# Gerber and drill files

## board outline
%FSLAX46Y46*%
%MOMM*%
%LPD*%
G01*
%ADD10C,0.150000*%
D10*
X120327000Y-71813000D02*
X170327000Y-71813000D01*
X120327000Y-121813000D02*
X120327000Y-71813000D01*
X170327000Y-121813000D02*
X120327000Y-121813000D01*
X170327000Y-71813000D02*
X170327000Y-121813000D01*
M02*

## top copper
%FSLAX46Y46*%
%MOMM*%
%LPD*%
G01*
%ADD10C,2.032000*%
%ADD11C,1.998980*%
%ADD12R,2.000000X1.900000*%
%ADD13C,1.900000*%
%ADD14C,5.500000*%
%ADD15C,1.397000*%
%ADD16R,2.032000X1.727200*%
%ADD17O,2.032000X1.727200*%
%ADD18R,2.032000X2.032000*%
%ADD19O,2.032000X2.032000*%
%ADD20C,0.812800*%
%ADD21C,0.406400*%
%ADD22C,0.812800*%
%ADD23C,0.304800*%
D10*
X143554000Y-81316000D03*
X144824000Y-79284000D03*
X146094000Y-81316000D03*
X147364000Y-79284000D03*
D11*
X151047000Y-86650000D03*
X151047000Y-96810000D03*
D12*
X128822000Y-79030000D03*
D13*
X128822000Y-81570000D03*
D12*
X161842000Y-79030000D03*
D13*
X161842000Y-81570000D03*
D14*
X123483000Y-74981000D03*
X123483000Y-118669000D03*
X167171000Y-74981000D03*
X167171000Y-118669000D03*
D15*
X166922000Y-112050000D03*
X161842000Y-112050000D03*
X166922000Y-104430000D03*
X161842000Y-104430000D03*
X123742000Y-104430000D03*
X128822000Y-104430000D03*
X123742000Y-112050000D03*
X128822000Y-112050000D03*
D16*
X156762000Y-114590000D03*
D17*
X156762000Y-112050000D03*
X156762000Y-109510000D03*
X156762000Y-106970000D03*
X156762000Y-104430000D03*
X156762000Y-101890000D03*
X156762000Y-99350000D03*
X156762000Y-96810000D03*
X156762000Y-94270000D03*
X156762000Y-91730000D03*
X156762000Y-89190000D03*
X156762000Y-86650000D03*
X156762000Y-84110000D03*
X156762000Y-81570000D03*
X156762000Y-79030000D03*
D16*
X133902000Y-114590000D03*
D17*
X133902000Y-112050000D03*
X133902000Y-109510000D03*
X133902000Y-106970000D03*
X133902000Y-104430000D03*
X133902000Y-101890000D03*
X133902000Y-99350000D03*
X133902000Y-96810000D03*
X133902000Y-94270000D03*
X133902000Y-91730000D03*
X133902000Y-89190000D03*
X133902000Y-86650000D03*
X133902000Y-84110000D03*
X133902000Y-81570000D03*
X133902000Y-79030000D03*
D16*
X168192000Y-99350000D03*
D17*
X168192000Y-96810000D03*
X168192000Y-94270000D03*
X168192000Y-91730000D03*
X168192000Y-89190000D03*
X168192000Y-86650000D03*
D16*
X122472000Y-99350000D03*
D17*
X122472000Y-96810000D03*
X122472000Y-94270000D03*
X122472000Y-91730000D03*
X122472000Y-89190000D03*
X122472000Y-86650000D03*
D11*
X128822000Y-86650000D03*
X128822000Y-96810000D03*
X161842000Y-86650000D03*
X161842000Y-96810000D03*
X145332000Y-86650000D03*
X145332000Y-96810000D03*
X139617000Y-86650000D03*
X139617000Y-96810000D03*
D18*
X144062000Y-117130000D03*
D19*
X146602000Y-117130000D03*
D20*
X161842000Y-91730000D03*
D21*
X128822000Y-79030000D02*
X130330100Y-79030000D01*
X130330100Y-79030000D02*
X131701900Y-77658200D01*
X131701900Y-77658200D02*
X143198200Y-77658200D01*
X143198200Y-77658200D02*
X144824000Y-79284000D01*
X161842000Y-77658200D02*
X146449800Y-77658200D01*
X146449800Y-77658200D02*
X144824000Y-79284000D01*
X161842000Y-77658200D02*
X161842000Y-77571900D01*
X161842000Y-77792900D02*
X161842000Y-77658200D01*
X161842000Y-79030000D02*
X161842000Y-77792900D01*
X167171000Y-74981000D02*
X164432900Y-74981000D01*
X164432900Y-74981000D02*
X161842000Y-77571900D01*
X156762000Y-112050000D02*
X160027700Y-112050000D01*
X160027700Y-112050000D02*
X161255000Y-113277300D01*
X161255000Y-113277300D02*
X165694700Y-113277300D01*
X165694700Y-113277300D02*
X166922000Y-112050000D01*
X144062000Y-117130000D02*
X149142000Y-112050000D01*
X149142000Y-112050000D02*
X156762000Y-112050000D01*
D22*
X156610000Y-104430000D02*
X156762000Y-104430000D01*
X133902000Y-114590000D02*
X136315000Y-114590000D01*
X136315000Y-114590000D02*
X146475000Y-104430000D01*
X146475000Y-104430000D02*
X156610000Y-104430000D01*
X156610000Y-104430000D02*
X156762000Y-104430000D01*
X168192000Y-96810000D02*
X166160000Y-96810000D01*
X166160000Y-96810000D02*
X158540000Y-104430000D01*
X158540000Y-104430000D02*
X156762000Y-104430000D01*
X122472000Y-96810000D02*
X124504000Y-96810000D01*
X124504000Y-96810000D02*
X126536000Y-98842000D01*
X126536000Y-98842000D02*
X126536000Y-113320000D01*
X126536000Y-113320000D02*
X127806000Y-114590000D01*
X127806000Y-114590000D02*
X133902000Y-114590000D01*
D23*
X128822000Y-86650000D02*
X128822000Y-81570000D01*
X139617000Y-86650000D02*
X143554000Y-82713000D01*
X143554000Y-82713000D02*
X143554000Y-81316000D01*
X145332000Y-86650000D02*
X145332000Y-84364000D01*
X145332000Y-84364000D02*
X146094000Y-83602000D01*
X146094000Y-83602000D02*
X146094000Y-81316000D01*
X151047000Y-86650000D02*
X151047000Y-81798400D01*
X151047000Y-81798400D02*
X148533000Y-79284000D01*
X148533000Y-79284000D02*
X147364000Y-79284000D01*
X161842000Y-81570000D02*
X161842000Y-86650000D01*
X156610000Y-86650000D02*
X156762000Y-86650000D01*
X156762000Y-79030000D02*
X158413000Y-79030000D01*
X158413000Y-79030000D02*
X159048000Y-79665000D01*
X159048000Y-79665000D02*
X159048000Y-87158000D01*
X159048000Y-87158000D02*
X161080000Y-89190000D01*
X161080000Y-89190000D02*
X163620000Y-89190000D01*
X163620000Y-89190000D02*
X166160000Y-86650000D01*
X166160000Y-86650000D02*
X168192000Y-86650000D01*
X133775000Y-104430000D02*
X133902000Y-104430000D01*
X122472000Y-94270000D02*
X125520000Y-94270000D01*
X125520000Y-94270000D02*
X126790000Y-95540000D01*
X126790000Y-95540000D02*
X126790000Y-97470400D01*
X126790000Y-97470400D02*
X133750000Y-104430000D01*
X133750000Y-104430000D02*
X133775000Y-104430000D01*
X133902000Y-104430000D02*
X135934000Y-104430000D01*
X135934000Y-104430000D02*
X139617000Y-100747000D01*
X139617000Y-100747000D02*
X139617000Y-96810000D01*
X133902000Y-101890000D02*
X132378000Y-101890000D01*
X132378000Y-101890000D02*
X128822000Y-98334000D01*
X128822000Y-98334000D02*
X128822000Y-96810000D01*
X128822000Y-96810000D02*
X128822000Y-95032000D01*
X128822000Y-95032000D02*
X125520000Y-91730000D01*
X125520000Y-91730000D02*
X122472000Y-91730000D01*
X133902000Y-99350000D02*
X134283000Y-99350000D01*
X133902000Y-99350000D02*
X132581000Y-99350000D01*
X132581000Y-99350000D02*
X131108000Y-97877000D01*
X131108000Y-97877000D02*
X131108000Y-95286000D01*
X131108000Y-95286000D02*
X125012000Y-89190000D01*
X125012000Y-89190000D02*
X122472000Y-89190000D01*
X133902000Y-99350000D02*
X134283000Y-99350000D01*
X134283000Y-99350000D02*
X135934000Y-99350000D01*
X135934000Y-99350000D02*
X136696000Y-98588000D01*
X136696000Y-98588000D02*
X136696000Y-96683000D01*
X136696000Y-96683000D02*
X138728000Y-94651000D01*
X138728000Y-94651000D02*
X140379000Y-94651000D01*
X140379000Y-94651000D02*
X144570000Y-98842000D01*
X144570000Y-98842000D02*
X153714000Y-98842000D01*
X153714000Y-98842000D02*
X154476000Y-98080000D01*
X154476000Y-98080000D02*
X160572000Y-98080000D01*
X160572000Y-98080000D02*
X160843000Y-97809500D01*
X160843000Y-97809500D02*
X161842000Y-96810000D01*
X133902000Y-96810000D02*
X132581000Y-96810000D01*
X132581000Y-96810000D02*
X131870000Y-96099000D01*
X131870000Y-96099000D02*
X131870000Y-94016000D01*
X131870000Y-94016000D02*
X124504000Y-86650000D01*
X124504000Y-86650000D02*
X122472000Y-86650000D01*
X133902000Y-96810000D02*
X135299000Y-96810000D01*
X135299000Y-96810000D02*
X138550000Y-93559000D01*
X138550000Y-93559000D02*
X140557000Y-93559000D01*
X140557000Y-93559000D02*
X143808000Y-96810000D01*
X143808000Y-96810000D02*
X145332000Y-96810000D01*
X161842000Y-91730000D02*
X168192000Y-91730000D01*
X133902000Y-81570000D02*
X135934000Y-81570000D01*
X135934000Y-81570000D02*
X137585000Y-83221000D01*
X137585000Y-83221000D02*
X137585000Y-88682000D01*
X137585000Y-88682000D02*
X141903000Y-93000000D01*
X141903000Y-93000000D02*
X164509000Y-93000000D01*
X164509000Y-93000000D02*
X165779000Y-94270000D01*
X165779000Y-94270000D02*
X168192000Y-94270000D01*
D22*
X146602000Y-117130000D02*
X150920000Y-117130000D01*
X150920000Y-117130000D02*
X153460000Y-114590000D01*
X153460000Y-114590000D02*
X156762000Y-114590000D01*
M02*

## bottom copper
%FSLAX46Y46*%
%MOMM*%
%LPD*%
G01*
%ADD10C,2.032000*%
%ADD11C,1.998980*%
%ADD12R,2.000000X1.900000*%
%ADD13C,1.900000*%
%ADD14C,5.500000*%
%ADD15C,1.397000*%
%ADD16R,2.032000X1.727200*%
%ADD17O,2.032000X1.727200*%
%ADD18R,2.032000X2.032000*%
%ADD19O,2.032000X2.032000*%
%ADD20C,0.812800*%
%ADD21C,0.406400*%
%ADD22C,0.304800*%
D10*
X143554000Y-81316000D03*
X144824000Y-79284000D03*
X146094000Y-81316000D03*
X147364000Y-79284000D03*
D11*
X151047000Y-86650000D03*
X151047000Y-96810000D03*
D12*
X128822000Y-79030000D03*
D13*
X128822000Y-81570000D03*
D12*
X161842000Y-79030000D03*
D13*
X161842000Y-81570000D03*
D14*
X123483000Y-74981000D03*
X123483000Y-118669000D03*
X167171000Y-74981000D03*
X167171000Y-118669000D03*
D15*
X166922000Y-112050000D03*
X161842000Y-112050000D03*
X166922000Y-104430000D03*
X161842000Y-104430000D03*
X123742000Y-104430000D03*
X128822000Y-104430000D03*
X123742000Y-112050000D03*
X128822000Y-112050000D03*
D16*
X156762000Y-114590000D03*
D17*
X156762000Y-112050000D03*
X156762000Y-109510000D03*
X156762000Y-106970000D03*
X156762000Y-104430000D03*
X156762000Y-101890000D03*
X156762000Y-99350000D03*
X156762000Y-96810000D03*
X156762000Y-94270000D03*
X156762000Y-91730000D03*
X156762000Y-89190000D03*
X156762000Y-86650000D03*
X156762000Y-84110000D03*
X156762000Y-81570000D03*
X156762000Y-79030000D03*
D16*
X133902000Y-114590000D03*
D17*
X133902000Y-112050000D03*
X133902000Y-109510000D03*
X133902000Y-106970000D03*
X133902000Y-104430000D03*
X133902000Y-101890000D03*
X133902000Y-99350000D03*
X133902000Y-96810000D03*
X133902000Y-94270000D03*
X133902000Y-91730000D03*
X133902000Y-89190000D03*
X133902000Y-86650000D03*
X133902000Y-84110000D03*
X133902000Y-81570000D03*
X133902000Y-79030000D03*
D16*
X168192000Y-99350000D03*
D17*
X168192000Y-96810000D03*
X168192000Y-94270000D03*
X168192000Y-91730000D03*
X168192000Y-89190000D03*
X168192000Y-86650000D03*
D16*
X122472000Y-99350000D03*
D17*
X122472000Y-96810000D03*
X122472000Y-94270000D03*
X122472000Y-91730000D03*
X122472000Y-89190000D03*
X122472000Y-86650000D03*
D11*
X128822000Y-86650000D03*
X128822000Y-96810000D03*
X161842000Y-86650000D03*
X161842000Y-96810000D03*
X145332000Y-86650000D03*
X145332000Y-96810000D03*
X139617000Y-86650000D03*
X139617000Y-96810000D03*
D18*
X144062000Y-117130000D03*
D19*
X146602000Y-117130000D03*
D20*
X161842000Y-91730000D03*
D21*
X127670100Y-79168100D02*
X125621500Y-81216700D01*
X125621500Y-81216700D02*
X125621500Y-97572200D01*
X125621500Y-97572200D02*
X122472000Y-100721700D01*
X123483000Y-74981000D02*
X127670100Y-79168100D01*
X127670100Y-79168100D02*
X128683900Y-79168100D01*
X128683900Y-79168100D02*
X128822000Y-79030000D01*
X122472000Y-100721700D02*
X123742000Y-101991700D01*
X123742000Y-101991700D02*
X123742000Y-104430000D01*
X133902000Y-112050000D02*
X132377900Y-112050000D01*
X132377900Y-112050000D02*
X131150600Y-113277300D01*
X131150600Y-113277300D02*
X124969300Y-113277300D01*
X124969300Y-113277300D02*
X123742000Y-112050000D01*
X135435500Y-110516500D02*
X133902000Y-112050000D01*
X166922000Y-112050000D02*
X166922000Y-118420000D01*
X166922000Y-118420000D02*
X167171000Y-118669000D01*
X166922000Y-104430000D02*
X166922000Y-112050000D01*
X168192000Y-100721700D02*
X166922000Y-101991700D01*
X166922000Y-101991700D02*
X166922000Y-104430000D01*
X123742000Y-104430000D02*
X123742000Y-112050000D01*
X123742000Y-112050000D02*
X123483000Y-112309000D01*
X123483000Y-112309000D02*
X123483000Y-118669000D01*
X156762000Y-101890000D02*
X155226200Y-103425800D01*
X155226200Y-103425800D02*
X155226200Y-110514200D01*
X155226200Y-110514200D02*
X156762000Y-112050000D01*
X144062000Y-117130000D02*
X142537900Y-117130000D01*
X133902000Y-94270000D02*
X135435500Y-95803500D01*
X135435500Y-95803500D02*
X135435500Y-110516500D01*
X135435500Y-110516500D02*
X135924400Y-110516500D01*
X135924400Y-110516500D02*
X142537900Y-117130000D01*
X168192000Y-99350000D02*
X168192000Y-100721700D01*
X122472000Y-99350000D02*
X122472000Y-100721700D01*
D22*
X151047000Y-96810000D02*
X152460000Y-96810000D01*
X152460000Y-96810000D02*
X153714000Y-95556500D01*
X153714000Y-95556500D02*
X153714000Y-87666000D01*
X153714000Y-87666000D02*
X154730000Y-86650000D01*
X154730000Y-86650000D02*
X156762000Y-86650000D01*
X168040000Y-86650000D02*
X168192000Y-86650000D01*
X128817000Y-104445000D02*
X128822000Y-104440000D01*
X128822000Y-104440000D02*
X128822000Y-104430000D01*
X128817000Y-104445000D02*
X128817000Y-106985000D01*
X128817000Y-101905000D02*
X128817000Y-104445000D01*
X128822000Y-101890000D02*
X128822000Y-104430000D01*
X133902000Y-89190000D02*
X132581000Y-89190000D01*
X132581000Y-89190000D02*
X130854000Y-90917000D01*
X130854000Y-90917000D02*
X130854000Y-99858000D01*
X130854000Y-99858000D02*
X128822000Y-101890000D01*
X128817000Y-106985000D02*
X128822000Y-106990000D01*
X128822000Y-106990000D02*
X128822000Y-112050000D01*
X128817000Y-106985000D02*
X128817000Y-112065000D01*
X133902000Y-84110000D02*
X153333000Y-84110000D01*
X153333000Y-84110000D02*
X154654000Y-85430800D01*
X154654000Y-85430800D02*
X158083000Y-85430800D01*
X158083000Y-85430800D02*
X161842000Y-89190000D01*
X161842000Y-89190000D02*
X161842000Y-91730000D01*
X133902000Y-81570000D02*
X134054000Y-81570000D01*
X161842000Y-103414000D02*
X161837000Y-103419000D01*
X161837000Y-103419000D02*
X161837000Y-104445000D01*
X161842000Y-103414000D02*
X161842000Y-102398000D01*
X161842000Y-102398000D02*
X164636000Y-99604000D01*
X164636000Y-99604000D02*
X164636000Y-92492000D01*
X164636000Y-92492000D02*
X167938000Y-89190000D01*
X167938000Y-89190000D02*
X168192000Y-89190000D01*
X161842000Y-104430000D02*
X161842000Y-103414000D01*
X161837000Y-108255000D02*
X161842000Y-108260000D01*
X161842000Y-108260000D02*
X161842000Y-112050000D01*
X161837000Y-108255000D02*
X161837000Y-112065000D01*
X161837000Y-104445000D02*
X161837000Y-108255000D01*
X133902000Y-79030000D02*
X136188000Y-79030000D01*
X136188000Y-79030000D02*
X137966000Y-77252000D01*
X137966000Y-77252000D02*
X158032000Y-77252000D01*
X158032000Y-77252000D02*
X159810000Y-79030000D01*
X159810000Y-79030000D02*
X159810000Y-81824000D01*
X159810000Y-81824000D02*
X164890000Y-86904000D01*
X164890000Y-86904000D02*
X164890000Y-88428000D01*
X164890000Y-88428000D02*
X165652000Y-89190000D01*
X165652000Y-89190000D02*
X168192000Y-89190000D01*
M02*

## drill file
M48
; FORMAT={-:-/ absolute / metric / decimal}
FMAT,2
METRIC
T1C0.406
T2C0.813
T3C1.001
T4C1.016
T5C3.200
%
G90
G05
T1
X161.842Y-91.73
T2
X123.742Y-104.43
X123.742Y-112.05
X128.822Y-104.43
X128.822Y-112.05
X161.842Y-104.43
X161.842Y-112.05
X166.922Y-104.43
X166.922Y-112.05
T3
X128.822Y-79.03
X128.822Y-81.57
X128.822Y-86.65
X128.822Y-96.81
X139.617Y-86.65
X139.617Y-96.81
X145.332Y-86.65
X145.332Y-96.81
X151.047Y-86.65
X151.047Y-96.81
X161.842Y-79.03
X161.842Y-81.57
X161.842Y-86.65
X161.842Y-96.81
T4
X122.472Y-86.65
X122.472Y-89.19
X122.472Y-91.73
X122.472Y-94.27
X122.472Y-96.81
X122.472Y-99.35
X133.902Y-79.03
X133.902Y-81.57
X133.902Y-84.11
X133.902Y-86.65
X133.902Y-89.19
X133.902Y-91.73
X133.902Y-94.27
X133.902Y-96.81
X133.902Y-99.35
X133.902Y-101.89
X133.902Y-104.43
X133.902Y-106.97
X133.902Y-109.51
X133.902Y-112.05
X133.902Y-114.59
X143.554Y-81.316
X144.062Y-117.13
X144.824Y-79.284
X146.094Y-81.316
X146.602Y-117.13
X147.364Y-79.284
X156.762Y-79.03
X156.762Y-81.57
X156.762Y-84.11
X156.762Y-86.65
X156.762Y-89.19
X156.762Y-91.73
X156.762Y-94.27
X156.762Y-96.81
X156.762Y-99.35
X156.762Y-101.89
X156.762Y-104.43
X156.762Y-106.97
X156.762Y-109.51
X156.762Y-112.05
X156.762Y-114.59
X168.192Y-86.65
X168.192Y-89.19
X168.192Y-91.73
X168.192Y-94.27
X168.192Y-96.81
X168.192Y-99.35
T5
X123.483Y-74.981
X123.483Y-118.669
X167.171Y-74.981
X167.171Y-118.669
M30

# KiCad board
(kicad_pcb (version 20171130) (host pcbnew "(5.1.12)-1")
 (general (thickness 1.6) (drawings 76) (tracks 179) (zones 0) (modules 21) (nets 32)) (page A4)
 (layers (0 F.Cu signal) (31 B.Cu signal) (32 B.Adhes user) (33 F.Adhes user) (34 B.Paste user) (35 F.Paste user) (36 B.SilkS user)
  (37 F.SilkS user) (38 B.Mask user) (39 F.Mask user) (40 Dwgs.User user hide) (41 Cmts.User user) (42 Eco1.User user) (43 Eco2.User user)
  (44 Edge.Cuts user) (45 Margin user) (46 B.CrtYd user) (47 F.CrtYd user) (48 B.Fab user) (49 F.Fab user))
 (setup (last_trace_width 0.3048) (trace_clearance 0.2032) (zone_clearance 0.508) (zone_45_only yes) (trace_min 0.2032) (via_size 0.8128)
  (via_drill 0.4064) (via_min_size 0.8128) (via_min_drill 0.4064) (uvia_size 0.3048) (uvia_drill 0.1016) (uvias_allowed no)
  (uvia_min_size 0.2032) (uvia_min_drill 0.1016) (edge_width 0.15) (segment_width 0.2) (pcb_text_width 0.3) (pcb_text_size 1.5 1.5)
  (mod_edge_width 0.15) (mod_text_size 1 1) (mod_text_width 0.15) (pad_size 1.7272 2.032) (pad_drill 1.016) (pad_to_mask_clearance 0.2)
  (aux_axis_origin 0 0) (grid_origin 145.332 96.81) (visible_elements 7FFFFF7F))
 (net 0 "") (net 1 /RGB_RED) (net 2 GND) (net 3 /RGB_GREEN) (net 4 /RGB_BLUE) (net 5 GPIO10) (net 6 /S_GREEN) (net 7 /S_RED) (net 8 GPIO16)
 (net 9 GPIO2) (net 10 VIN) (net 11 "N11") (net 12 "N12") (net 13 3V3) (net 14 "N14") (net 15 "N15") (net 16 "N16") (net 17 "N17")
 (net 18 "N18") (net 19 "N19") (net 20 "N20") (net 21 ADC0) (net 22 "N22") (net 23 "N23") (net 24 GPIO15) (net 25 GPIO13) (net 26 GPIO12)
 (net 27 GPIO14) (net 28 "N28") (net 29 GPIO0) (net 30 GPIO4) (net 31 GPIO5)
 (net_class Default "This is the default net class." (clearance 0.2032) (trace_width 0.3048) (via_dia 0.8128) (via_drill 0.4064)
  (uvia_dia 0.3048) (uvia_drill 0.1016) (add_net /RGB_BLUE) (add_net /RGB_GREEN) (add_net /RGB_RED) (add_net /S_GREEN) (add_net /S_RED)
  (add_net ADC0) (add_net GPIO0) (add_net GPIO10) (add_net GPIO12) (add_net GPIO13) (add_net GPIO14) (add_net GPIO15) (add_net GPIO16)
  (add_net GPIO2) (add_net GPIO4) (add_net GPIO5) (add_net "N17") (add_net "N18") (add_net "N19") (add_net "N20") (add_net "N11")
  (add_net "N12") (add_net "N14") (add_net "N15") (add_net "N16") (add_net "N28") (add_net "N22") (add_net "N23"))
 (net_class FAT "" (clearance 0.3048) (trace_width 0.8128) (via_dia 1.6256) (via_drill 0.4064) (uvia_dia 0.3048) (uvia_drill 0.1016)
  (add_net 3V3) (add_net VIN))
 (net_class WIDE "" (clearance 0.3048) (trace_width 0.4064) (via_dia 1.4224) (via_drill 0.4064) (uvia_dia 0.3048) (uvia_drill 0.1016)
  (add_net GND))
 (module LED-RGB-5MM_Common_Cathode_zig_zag (layer F.Cu) (at 143.554 80.3 90)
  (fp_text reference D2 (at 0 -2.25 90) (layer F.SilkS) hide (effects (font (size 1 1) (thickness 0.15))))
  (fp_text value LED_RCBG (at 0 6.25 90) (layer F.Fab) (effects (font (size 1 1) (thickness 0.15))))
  (pad 1 thru_hole circle (at -1.016 0 90) (size 2.032 2.032) (drill 1.016) (layers *.Cu *.Mask F.SilkS) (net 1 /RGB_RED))
  (pad 2 thru_hole circle (at 1.016 1.27 90) (size 2.032 2.032) (drill 1.016) (layers *.Cu *.Mask F.SilkS) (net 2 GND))
  (pad 3 thru_hole circle (at -1.016 2.54 90) (size 2.032 2.032) (drill 1.016) (layers *.Cu *.Mask F.SilkS) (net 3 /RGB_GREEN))
  (pad 4 thru_hole circle (at 1.016 3.81 90) (size 2.032 2.032) (drill 1.016) (layers *.Cu *.Mask F.SilkS) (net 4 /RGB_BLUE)))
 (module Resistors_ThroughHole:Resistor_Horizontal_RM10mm (layer F.Cu) (at 151.047 86.65 270)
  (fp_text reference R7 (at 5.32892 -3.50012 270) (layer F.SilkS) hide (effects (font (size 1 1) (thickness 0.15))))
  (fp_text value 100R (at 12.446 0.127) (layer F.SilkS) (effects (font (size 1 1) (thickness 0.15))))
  (pad 1 thru_hole circle (at 0 0 270) (size 1.99898 1.99898) (drill 1.00076) (layers *.Cu *.SilkS *.Mask) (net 4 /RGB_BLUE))
  (pad 2 thru_hole circle (at 10.16 0 270) (size 1.99898 1.99898) (drill 1.00076) (layers *.Cu *.SilkS *.Mask) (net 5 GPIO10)))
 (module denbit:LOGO (layer B.Cu) (at 145.332 103.16 180)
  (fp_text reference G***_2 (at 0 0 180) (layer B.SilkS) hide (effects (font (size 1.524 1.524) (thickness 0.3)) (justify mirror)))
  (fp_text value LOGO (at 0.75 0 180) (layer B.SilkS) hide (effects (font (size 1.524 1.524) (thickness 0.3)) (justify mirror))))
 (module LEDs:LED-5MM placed (layer F.Cu) (at 128.822 79.03 270)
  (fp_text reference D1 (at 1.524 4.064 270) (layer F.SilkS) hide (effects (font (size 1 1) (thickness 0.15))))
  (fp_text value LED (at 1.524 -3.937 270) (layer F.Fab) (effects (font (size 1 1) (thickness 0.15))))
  (pad 1 thru_hole rect (at 0 0) (size 2 1.9) (drill 1.00076) (layers *.Cu *.Mask F.SilkS) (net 2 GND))
  (pad 2 thru_hole circle (at 2.54 0 270) (size 1.9 1.9) (drill 1.00076) (layers *.Cu *.Mask F.SilkS) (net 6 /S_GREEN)))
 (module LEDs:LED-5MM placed (layer F.Cu) (at 161.842 79.03 270)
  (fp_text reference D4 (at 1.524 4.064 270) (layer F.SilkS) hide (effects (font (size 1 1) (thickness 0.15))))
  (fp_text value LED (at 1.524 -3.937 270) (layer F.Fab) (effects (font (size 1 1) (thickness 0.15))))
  (pad 1 thru_hole rect (at 0 0) (size 2 1.9) (drill 1.00076) (layers *.Cu *.Mask F.SilkS) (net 2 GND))
  (pad 2 thru_hole circle (at 2.54 0 270) (size 1.9 1.9) (drill 1.00076) (layers *.Cu *.Mask F.SilkS) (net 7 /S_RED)))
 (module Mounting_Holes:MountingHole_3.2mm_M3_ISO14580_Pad (layer F.Cu) (at 123.483 74.981 270)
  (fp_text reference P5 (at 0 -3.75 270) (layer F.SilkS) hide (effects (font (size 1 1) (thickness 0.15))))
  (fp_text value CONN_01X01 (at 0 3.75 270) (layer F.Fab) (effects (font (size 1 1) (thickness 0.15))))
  (pad 1 thru_hole circle (at 0 0 270) (size 5.5 5.5) (drill 3.2) (layers *.Cu *.Mask F.SilkS) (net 2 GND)))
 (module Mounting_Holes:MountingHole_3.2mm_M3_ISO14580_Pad (layer F.Cu) (at 123.483 118.669 270)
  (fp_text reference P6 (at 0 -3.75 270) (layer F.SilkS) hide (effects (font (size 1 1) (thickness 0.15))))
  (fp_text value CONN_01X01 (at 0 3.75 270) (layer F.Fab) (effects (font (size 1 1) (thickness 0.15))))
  (pad 1 thru_hole circle (at 0 0 270) (size 5.5 5.5) (drill 3.2) (layers *.Cu *.Mask F.SilkS) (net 2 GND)))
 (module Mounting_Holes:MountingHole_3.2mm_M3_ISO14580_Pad (layer F.Cu) (at 167.171 74.981 270)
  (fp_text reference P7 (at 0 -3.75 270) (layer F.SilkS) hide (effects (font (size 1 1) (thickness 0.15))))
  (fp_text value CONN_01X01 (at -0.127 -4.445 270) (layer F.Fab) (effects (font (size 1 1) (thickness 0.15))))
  (pad 1 thru_hole circle (at 0 0 270) (size 5.5 5.5) (drill 3.2) (layers *.Cu *.Mask F.SilkS) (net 2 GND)))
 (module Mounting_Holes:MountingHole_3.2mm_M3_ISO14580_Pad (layer F.Cu) (at 167.171 118.669 270)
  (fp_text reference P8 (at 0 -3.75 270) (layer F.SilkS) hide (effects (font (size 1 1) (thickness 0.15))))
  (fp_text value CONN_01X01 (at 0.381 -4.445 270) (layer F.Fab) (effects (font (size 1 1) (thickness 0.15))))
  (pad 1 thru_hole circle (at 0 0 270) (size 5.5 5.5) (drill 3.2) (layers *.Cu *.Mask F.SilkS) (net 2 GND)))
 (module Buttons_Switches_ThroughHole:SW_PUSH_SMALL (layer F.Cu) (at 164.382 108.24 270)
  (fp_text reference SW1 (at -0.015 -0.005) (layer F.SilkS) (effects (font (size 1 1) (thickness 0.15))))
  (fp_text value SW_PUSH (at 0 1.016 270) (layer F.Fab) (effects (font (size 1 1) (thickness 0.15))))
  (pad 1 thru_hole circle (at 3.81 -2.54 270) (size 1.397 1.397) (drill 0.8128) (layers *.Cu *.Mask F.SilkS) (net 2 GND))
  (pad 2 thru_hole circle (at 3.81 2.54 270) (size 1.397 1.397) (drill 0.8128) (layers *.Cu *.Mask F.SilkS) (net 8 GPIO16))
  (pad 1 thru_hole circle (at -3.81 -2.54 270) (size 1.397 1.397) (drill 0.8128) (layers *.Cu *.Mask F.SilkS) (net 2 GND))
  (pad 2 thru_hole circle (at -3.81 2.54 270) (size 1.397 1.397) (drill 0.8128) (layers *.Cu *.Mask F.SilkS) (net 8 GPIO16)))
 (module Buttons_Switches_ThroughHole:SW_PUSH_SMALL (layer F.Cu) (at 126.282 108.24 90)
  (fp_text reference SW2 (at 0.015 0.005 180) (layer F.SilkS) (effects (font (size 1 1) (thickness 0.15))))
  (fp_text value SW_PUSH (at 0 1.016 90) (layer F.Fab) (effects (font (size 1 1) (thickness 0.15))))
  (pad 1 thru_hole circle (at 3.81 -2.54 90) (size 1.397 1.397) (drill 0.8128) (layers *.Cu *.Mask F.SilkS) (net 2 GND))
  (pad 2 thru_hole circle (at 3.81 2.54 90) (size 1.397 1.397) (drill 0.8128) (layers *.Cu *.Mask F.SilkS) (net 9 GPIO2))
  (pad 1 thru_hole circle (at -3.81 -2.54 90) (size 1.397 1.397) (drill 0.8128) (layers *.Cu *.Mask F.SilkS) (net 2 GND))
  (pad 2 thru_hole circle (at -3.81 2.54 90) (size 1.397 1.397) (drill 0.8128) (layers *.Cu *.Mask F.SilkS) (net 9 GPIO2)))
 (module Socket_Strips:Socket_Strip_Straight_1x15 (layer B.Cu) (at 156.762 114.59 90)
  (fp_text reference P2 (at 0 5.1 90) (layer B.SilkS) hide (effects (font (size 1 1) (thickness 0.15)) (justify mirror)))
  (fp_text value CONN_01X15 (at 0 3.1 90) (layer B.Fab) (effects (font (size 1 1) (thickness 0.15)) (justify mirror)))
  (pad 1 thru_hole rect (at 0 0 90) (size 1.7272 2.032) (drill 1.016) (layers *.Cu *.Mask B.SilkS) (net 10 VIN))
  (pad 2 thru_hole oval (at 2.54 0 90) (size 1.7272 2.032) (drill 1.016) (layers *.Cu *.Mask B.SilkS) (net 2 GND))
  (pad 3 thru_hole oval (at 5.08 0 90) (size 1.7272 2.032) (drill 1.016) (layers *.Cu *.Mask B.SilkS) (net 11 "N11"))
  (pad 4 thru_hole oval (at 7.62 0 90) (size 1.7272 2.032) (drill 1.016) (layers *.Cu *.Mask B.SilkS) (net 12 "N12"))
  (pad 5 thru_hole oval (at 10.16 0 90) (size 1.7272 2.032) (drill 1.016) (layers *.Cu *.Mask B.SilkS) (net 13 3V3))
  (pad 6 thru_hole oval (at 12.7 0 90) (size 1.7272 2.032) (drill 1.016) (layers *.Cu *.Mask B.SilkS) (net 2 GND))
  (pad 7 thru_hole oval (at 15.24 0 90) (size 1.7272 2.032) (drill 1.016) (layers *.Cu *.Mask B.SilkS) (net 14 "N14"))
  (pad 8 thru_hole oval (at 17.78 0 90) (size 1.7272 2.032) (drill 1.016) (layers *.Cu *.Mask B.SilkS) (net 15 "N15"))
  (pad 9 thru_hole oval (at 20.32 0 90) (size 1.7272 2.032) (drill 1.016) (layers *.Cu *.Mask B.SilkS) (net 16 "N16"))
  (pad 10 thru_hole oval (at 22.86 0 90) (size 1.7272 2.032) (drill 1.016) (layers *.Cu *.Mask B.SilkS) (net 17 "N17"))
  (pad 11 thru_hole oval (at 25.4 0 90) (size 1.7272 2.032) (drill 1.016) (layers *.Cu *.Mask B.SilkS) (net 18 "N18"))
  (pad 12 thru_hole oval (at 27.94 0 90) (size 1.7272 2.032) (drill 1.016) (layers *.Cu *.Mask B.SilkS) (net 5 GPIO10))
  (pad 13 thru_hole oval (at 30.48 0 90) (size 1.7272 2.032) (drill 1.016) (layers *.Cu *.Mask B.SilkS) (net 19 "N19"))
  (pad 14 thru_hole oval (at 33.02 0 90) (size 1.7272 2.032) (drill 1.016) (layers *.Cu *.Mask B.SilkS) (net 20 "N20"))
  (pad 15 thru_hole oval (at 35.56 0 90) (size 1.7272 2.032) (drill 1.016) (layers *.Cu *.Mask B.SilkS) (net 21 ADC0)))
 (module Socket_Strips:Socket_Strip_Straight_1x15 (layer B.Cu) (at 133.902 114.59 90)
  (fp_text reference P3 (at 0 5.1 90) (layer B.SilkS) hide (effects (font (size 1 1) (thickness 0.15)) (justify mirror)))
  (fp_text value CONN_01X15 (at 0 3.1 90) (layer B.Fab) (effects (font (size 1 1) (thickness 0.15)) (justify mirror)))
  (pad 1 thru_hole rect (at 0 0 90) (size 1.7272 2.032) (drill 1.016) (layers *.Cu *.Mask B.SilkS) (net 13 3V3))
  (pad 2 thru_hole oval (at 2.54 0 90) (size 1.7272 2.032) (drill 1.016) (layers *.Cu *.Mask B.SilkS) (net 2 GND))
  (pad 3 thru_hole oval (at 5.08 0 90) (size 1.7272 2.032) (drill 1.016) (layers *.Cu *.Mask B.SilkS) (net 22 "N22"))
  (pad 4 thru_hole oval (at 7.62 0 90) (size 1.7272 2.032) (drill 1.016) (layers *.Cu *.Mask B.SilkS) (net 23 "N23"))
  (pad 5 thru_hole oval (at 10.16 0 90) (size 1.7272 2.032) (drill 1.016) (layers *.Cu *.Mask B.SilkS) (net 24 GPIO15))
  (pad 6 thru_hole oval (at 12.7 0 90) (size 1.7272 2.032) (drill 1.016) (layers *.Cu *.Mask B.SilkS) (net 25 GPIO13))
  (pad 7 thru_hole oval (at 15.24 0 90) (size 1.7272 2.032) (drill 1.016) (layers *.Cu *.Mask B.SilkS) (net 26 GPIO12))
  (pad 8 thru_hole oval (at 17.78 0 90) (size 1.7272 2.032) (drill 1.016) (layers *.Cu *.Mask B.SilkS) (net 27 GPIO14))
  (pad 9 thru_hole oval (at 20.32 0 90) (size 1.7272 2.032) (drill 1.016) (layers *.Cu *.Mask B.SilkS) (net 2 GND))
  (pad 10 thru_hole oval (at 22.86 0 90) (size 1.7272 2.032) (drill 1.016) (layers *.Cu *.Mask B.SilkS) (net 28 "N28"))
  (pad 11 thru_hole oval (at 25.4 0 90) (size 1.7272 2.032) (drill 1.016) (layers *.Cu *.Mask B.SilkS) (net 9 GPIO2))
  (pad 12 thru_hole oval (at 27.94 0 90) (size 1.7272 2.032) (drill 1.016) (layers *.Cu *.Mask B.SilkS) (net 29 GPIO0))
  (pad 13 thru_hole oval (at 30.48 0 90) (size 1.7272 2.032) (drill 1.016) (layers *.Cu *.Mask B.SilkS) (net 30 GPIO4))
  (pad 14 thru_hole oval (at 33.02 0 90) (size 1.7272 2.032) (drill 1.016) (layers *.Cu *.Mask B.SilkS) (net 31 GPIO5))
  (pad 15 thru_hole oval (at 35.56 0 90) (size 1.7272 2.032) (drill 1.016) (layers *.Cu *.Mask B.SilkS) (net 8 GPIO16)))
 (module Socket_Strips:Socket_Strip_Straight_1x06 (layer F.Cu) (at 168.192 99.35 90)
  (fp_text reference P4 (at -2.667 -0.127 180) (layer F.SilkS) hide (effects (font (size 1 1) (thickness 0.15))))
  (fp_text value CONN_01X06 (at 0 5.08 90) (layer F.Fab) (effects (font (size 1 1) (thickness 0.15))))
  (pad 1 thru_hole rect (at 0 0 90) (size 1.7272 2.032) (drill 1.016) (layers *.Cu *.Mask F.SilkS) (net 2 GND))
  (pad 2 thru_hole oval (at 2.54 0 90) (size 1.7272 2.032) (drill 1.016) (layers *.Cu *.Mask F.SilkS) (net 13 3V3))
  (pad 3 thru_hole oval (at 5.08 0 90) (size 1.7272 2.032) (drill 1.016) (layers *.Cu *.Mask F.SilkS) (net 31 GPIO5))
  (pad 4 thru_hole oval (at 7.62 0 90) (size 1.7272 2.032) (drill 1.016) (layers *.Cu *.Mask F.SilkS) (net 30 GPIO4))
  (pad 5 thru_hole oval (at 10.16 0 90) (size 1.7272 2.032) (drill 1.016) (layers *.Cu *.Mask F.SilkS) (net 8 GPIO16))
  (pad 6 thru_hole oval (at 12.7 0 90) (size 1.7272 2.032) (drill 1.016) (layers *.Cu *.Mask F.SilkS) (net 21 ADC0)))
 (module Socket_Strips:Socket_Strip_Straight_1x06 (layer F.Cu) (at 122.472 99.35 90)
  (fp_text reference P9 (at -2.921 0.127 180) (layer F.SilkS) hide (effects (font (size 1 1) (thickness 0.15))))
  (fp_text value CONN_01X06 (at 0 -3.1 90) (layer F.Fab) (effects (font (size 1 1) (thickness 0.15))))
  (pad 1 thru_hole rect (at 0 0 90) (size 1.7272 2.032) (drill 1.016) (layers *.Cu *.Mask F.SilkS) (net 2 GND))
  (pad 2 thru_hole oval (at 2.54 0 90) (size 1.7272 2.032) (drill 1.016) (layers *.Cu *.Mask F.SilkS) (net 13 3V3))
  (pad 3 thru_hole oval (at 5.08 0 90) (size 1.7272 2.032) (drill 1.016) (layers *.Cu *.Mask F.SilkS) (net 24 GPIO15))
  (pad 4 thru_hole oval (at 7.62 0 90) (size 1.7272 2.032) (drill 1.016) (layers *.Cu *.Mask F.SilkS) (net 25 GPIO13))
  (pad 5 thru_hole oval (at 10.16 0 90) (size 1.7272 2.032) (drill 1.016) (layers *.Cu *.Mask F.SilkS) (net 26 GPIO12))
  (pad 6 thru_hole oval (at 12.7 0 90) (size 1.7272 2.032) (drill 1.016) (layers *.Cu *.Mask F.SilkS) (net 27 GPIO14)))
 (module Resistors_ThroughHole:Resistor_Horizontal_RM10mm (layer F.Cu) (at 128.822 86.65 270)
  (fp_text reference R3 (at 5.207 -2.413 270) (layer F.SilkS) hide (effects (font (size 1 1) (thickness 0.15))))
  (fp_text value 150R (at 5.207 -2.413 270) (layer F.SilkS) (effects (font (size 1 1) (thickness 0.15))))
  (pad 1 thru_hole circle (at 0 0 270) (size 1.99898 1.99898) (drill 1.00076) (layers *.Cu *.SilkS *.Mask) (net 6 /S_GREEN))
  (pad 2 thru_hole circle (at 10.16 0 270) (size 1.99898 1.99898) (drill 1.00076) (layers *.Cu *.SilkS *.Mask) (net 25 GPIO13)))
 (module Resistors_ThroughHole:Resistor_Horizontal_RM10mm (layer F.Cu) (at 161.842 86.65 270)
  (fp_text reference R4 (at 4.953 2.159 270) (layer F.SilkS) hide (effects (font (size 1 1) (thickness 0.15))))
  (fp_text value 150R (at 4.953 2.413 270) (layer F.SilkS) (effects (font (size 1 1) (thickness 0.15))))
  (pad 1 thru_hole circle (at 0 0 270) (size 1.99898 1.99898) (drill 1.00076) (layers *.Cu *.SilkS *.Mask) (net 7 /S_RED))
  (pad 2 thru_hole circle (at 10.16 0 270) (size 1.99898 1.99898) (drill 1.00076) (layers *.Cu *.SilkS *.Mask) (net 26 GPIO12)))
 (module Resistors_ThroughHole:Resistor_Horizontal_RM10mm (layer F.Cu) (at 145.332 86.65 270)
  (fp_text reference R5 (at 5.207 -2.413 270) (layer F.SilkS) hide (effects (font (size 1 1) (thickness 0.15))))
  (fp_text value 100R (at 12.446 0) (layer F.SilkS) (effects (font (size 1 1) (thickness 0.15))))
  (pad 1 thru_hole circle (at 0 0 270) (size 1.99898 1.99898) (drill 1.00076) (layers *.Cu *.SilkS *.Mask) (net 3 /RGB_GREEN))
  (pad 2 thru_hole circle (at 10.16 0 270) (size 1.99898 1.99898) (drill 1.00076) (layers *.Cu *.SilkS *.Mask) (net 27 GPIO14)))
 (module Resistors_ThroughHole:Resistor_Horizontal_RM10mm (layer F.Cu) (at 139.617 86.65 270)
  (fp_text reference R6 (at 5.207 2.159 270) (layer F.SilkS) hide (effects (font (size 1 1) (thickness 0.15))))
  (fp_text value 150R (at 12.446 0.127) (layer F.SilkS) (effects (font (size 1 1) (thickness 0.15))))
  (pad 1 thru_hole circle (at 0 0 270) (size 1.99898 1.99898) (drill 1.00076) (layers *.Cu *.SilkS *.Mask) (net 1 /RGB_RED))
  (pad 2 thru_hole circle (at 10.16 0 270) (size 1.99898 1.99898) (drill 1.00076) (layers *.Cu *.SilkS *.Mask) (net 24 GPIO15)))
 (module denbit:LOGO (layer F.Cu) (at 145.332 105.7)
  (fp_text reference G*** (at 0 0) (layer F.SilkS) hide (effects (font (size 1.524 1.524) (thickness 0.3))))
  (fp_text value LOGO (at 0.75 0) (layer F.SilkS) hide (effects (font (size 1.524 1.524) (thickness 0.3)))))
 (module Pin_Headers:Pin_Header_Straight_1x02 (layer F.Cu) (at 144.062 117.13 90)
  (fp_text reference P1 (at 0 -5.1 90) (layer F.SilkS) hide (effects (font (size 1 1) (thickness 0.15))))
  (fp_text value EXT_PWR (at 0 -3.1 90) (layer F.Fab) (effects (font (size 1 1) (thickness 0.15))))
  (pad 1 thru_hole rect (at 0 0 90) (size 2.032 2.032) (drill 1.016) (layers *.Cu *.Mask F.SilkS) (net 2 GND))
  (pad 2 thru_hole oval (at 0 2.54 90) (size 2.032 2.032) (drill 1.016) (layers *.Cu *.Mask F.SilkS) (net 10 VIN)))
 (gr_line (start 120.327 71.813) (end 170.327 71.813) (angle 90) (layer Edge.Cuts) (width 0.15))
 (gr_line (start 120.327 121.813) (end 120.327 71.813) (angle 90) (layer Edge.Cuts) (width 0.15))
 (gr_line (start 170.327 121.813) (end 120.327 121.813) (angle 90) (layer Edge.Cuts) (width 0.15))
 (gr_line (start 170.327 71.813) (end 170.327 121.813) (angle 90) (layer Edge.Cuts) (width 0.15))
 (segment (start 128.822 79.03) (end 130.3301 79.03) (width 0.4064) (layer F.Cu) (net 2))
 (segment (start 130.3301 79.03) (end 131.7019 77.6582) (width 0.4064) (layer F.Cu) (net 2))
 (segment (start 131.7019 77.6582) (end 143.1982 77.6582) (width 0.4064) (layer F.Cu) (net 2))
 (segment (start 143.1982 77.6582) (end 144.824 79.284) (width 0.4064) (layer F.Cu) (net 2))
 (segment (start 161.842 77.6582) (end 146.4498 77.6582) (width 0.4064) (layer F.Cu) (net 2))
 (segment (start 146.4498 77.6582) (end 144.824 79.284) (width 0.4064) (layer F.Cu) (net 2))
 (segment (start 161.842 77.6582) (end 161.842 77.5719) (width 0.4064) (layer F.Cu) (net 2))
 (segment (start 161.842 77.7929) (end 161.842 77.6582) (width 0.4064) (layer F.Cu) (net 2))
 (segment (start 161.842 79.03) (end 161.842 77.7929) (width 0.4064) (layer F.Cu) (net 2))
 (segment (start 127.6701 79.1681) (end 125.6215 81.2167) (width 0.4064) (layer B.Cu) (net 2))
 (segment (start 125.6215 81.2167) (end 125.6215 97.5722) (width 0.4064) (layer B.Cu) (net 2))
 (segment (start 125.6215 97.5722) (end 122.472 100.7217) (width 0.4064) (layer B.Cu) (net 2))
 (segment (start 123.483 74.981) (end 127.6701 79.1681) (width 0.4064) (layer B.Cu) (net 2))
 (segment (start 127.6701 79.1681) (end 128.6839 79.1681) (width 0.4064) (layer B.Cu) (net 2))
 (segment (start 128.6839 79.1681) (end 128.822 79.03) (width 0.4064) (layer B.Cu) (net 2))
 (segment (start 122.472 100.7217) (end 123.742 101.9917) (width 0.4064) (layer B.Cu) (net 2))
 (segment (start 123.742 101.9917) (end 123.742 104.43) (width 0.4064) (layer B.Cu) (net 2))
 (segment (start 167.171 74.981) (end 164.4329 74.981) (width 0.4064) (layer F.Cu) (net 2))
 (segment (start 164.4329 74.981) (end 161.842 77.5719) (width 0.4064) (layer F.Cu) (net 2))
 (segment (start 133.902 112.05) (end 132.3779 112.05) (width 0.4064) (layer B.Cu) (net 2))
 (segment (start 132.3779 112.05) (end 131.1506 113.2773) (width 0.4064) (layer B.Cu) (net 2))
 (segment (start 131.1506 113.2773) (end 124.9693 113.2773) (width 0.4064) (layer B.Cu) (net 2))
 (segment (start 124.9693 113.2773) (end 123.742 112.05) (width 0.4064) (layer B.Cu) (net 2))
 (segment (start 135.4355 110.5165) (end 133.902 112.05) (width 0.4064) (layer B.Cu) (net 2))
 (segment (start 166.922 112.05) (end 166.922 118.42) (width 0.4064) (layer B.Cu) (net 2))
 (segment (start 166.922 118.42) (end 167.171 118.669) (width 0.4064) (layer B.Cu) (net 2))
 (segment (start 166.922 104.43) (end 166.922 112.05) (width 0.4064) (layer B.Cu) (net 2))
 (segment (start 168.192 100.7217) (end 166.922 101.9917) (width 0.4064) (layer B.Cu) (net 2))
 (segment (start 166.922 101.9917) (end 166.922 104.43) (width 0.4064) (layer B.Cu) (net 2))
 (segment (start 123.742 104.43) (end 123.742 112.05) (width 0.4064) (layer B.Cu) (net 2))
 (segment (start 123.742 112.05) (end 123.483 112.309) (width 0.4064) (layer B.Cu) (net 2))
 (segment (start 123.483 112.309) (end 123.483 118.669) (width 0.4064) (layer B.Cu) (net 2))
 (segment (start 156.762 112.05) (end 160.0277 112.05) (width 0.4064) (layer F.Cu) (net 2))
 (segment (start 160.0277 112.05) (end 161.255 113.2773) (width 0.4064) (layer F.Cu) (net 2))
 (segment (start 161.255 113.2773) (end 165.6947 113.2773) (width 0.4064) (layer F.Cu) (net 2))
 (segment (start 165.6947 113.2773) (end 166.922 112.05) (width 0.4064) (layer F.Cu) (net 2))
 (segment (start 144.062 117.13) (end 149.142 112.05) (width 0.4064) (layer F.Cu) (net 2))
 (segment (start 149.142 112.05) (end 156.762 112.05) (width 0.4064) (layer F.Cu) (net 2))
 (segment (start 156.762 101.89) (end 155.2262 103.4258) (width 0.4064) (layer B.Cu) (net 2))
 (segment (start 155.2262 103.4258) (end 155.2262 110.5142) (width 0.4064) (layer B.Cu) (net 2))
 (segment (start 155.2262 110.5142) (end 156.762 112.05) (width 0.4064) (layer B.Cu) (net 2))
 (segment (start 144.062 117.13) (end 142.5379 117.13) (width 0.4064) (layer B.Cu) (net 2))
 (segment (start 133.902 94.27) (end 135.4355 95.8035) (width 0.4064) (layer B.Cu) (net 2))
 (segment (start 135.4355 95.8035) (end 135.4355 110.5165) (width 0.4064) (layer B.Cu) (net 2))
 (segment (start 135.4355 110.5165) (end 135.9244 110.5165) (width 0.4064) (layer B.Cu) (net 2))
 (segment (start 135.9244 110.5165) (end 142.5379 117.13) (width 0.4064) (layer B.Cu) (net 2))
 (segment (start 168.192 99.35) (end 168.192 100.7217) (width 0.4064) (layer B.Cu) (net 2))
 (segment (start 122.472 99.35) (end 122.472 100.7217) (width 0.4064) (layer B.Cu) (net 2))
 (segment (start 156.61 104.43) (end 156.762 104.43) (width 0.8128) (layer F.Cu) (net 13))
 (segment (start 133.902 114.59) (end 136.315 114.59) (width 0.8128) (layer F.Cu) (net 13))
 (segment (start 136.315 114.59) (end 146.475 104.43) (width 0.8128) (layer F.Cu) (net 13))
 (segment (start 146.475 104.43) (end 156.61 104.43) (width 0.8128) (layer F.Cu) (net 13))
 (segment (start 156.61 104.43) (end 156.762 104.43) (width 0.8128) (layer F.Cu) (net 13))
 (segment (start 168.192 96.81) (end 166.16 96.81) (width 0.8128) (layer F.Cu) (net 13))
 (segment (start 166.16 96.81) (end 158.54 104.43) (width 0.8128) (layer F.Cu) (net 13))
 (segment (start 158.54 104.43) (end 156.762 104.43) (width 0.8128) (layer F.Cu) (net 13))
 (segment (start 122.472 96.81) (end 124.504 96.81) (width 0.8128) (layer F.Cu) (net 13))
 (segment (start 124.504 96.81) (end 126.536 98.842) (width 0.8128) (layer F.Cu) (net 13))
 (segment (start 126.536 98.842) (end 126.536 113.32) (width 0.8128) (layer F.Cu) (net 13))
 (segment (start 126.536 113.32) (end 127.806 114.59) (width 0.8128) (layer F.Cu) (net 13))
 (segment (start 127.806 114.59) (end 133.902 114.59) (width 0.8128) (layer F.Cu) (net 13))
 (segment (start 128.822 86.65) (end 128.822 81.57) (width 0.3048) (layer F.Cu) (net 6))
 (segment (start 139.617 86.65) (end 143.554 82.713) (width 0.3048) (layer F.Cu) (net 1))
 (segment (start 143.554 82.713) (end 143.554 81.316) (width 0.3048) (layer F.Cu) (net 1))
 (segment (start 145.332 86.65) (end 145.332 84.364) (width 0.3048) (layer F.Cu) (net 3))
 (segment (start 145.332 84.364) (end 146.094 83.602) (width 0.3048) (layer F.Cu) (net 3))
 (segment (start 146.094 83.602) (end 146.094 81.316) (width 0.3048) (layer F.Cu) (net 3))
 (segment (start 151.047 86.65) (end 151.047 81.7984) (width 0.3048) (layer F.Cu) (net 4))
 (segment (start 151.047 81.7984) (end 148.533 79.284) (width 0.3048) (layer F.Cu) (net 4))
 (segment (start 148.533 79.284) (end 147.364 79.284) (width 0.3048) (layer F.Cu) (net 4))
 (segment (start 161.842 81.57) (end 161.842 86.65) (width 0.3048) (layer F.Cu) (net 7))
 (segment (start 156.61 86.65) (end 156.762 86.65) (width 0.3048) (layer F.Cu) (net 5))
 (segment (start 151.047 96.81) (end 152.46 96.81) (width 0.3048) (layer B.Cu) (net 5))
 (segment (start 152.46 96.81) (end 153.714 95.5565) (width 0.3048) (layer B.Cu) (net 5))
 (segment (start 153.714 95.5565) (end 153.714 87.666) (width 0.3048) (layer B.Cu) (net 5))
 (segment (start 153.714 87.666) (end 154.73 86.65) (width 0.3048) (layer B.Cu) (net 5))
 (segment (start 154.73 86.65) (end 156.762 86.65) (width 0.3048) (layer B.Cu) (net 5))
 (segment (start 168.04 86.65) (end 168.192 86.65) (width 0.3048) (layer B.Cu) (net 21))
 (segment (start 156.762 79.03) (end 158.413 79.03) (width 0.3048) (layer F.Cu) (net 21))
 (segment (start 158.413 79.03) (end 159.048 79.665) (width 0.3048) (layer F.Cu) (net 21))
 (segment (start 159.048 79.665) (end 159.048 87.158) (width 0.3048) (layer F.Cu) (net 21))
 (segment (start 159.048 87.158) (end 161.08 89.19) (width 0.3048) (layer F.Cu) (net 21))
 (segment (start 161.08 89.19) (end 163.62 89.19) (width 0.3048) (layer F.Cu) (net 21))
 (segment (start 163.62 89.19) (end 166.16 86.65) (width 0.3048) (layer F.Cu) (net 21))
 (segment (start 166.16 86.65) (end 168.192 86.65) (width 0.3048) (layer F.Cu) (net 21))
 (segment (start 133.775 104.43) (end 133.902 104.43) (width 0.3048) (layer F.Cu) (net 24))
 (segment (start 122.472 94.27) (end 125.52 94.27) (width 0.3048) (layer F.Cu) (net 24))
 (segment (start 125.52 94.27) (end 126.79 95.54) (width 0.3048) (layer F.Cu) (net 24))
 (segment (start 126.79 95.54) (end 126.79 97.4704) (width 0.3048) (layer F.Cu) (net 24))
 (segment (start 126.79 97.4704) (end 133.75 104.43) (width 0.3048) (layer F.Cu) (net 24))
 (segment (start 133.75 104.43) (end 133.775 104.43) (width 0.3048) (layer F.Cu) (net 24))
 (segment (start 133.902 104.43) (end 135.934 104.43) (width 0.3048) (layer F.Cu) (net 24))
 (segment (start 135.934 104.43) (end 139.617 100.747) (width 0.3048) (layer F.Cu) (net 24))
 (segment (start 139.617 100.747) (end 139.617 96.81) (width 0.3048) (layer F.Cu) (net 24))
 (segment (start 133.902 101.89) (end 132.378 101.89) (width 0.3048) (layer F.Cu) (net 25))
 (segment (start 132.378 101.89) (end 128.822 98.334) (width 0.3048) (layer F.Cu) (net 25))
 (segment (start 128.822 98.334) (end 128.822 96.81) (width 0.3048) (layer F.Cu) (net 25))
 (segment (start 128.822 96.81) (end 128.822 95.032) (width 0.3048) (layer F.Cu) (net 25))
 (segment (start 128.822 95.032) (end 125.52 91.73) (width 0.3048) (layer F.Cu) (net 25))
 (segment (start 125.52 91.73) (end 122.472 91.73) (width 0.3048) (layer F.Cu) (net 25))
 (segment (start 133.902 99.35) (end 134.283 99.35) (width 0.3048) (layer F.Cu) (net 26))
 (segment (start 133.902 99.35) (end 132.581 99.35) (width 0.3048) (layer F.Cu) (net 26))
 (segment (start 132.581 99.35) (end 131.108 97.877) (width 0.3048) (layer F.Cu) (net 26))
 (segment (start 131.108 97.877) (end 131.108 95.286) (width 0.3048) (layer F.Cu) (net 26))
 (segment (start 131.108 95.286) (end 125.012 89.19) (width 0.3048) (layer F.Cu) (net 26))
 (segment (start 125.012 89.19) (end 122.472 89.19) (width 0.3048) (layer F.Cu) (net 26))
 (segment (start 133.902 99.35) (end 134.283 99.35) (width 0.3048) (layer F.Cu) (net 26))
 (segment (start 134.283 99.35) (end 135.934 99.35) (width 0.3048) (layer F.Cu) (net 26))
 (segment (start 135.934 99.35) (end 136.696 98.588) (width 0.3048) (layer F.Cu) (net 26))
 (segment (start 136.696 98.588) (end 136.696 96.683) (width 0.3048) (layer F.Cu) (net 26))
 (segment (start 136.696 96.683) (end 138.728 94.651) (width 0.3048) (layer F.Cu) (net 26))
 (segment (start 138.728 94.651) (end 140.379 94.651) (width 0.3048) (layer F.Cu) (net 26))
 (segment (start 140.379 94.651) (end 144.57 98.842) (width 0.3048) (layer F.Cu) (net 26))
 (segment (start 144.57 98.842) (end 153.714 98.842) (width 0.3048) (layer F.Cu) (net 26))
 (segment (start 153.714 98.842) (end 154.476 98.08) (width 0.3048) (layer F.Cu) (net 26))
 (segment (start 154.476 98.08) (end 160.572 98.08) (width 0.3048) (layer F.Cu) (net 26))
 (segment (start 160.572 98.08) (end 160.843 97.8095) (width 0.3048) (layer F.Cu) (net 26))
 (segment (start 160.843 97.8095) (end 161.842 96.81) (width 0.3048) (layer F.Cu) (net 26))
 (segment (start 133.902 96.81) (end 132.581 96.81) (width 0.3048) (layer F.Cu) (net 27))
 (segment (start 132.581 96.81) (end 131.87 96.099) (width 0.3048) (layer F.Cu) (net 27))
 (segment (start 131.87 96.099) (end 131.87 94.016) (width 0.3048) (layer F.Cu) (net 27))
 (segment (start 131.87 94.016) (end 124.504 86.65) (width 0.3048) (layer F.Cu) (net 27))
 (segment (start 124.504 86.65) (end 122.472 86.65) (width 0.3048) (layer F.Cu) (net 27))
 (segment (start 133.902 96.81) (end 135.299 96.81) (width 0.3048) (layer F.Cu) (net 27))
 (segment (start 135.299 96.81) (end 138.55 93.559) (width 0.3048) (layer F.Cu) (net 27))
 (segment (start 138.55 93.559) (end 140.557 93.559) (width 0.3048) (layer F.Cu) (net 27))
 (segment (start 140.557 93.559) (end 143.808 96.81) (width 0.3048) (layer F.Cu) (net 27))
 (segment (start 143.808 96.81) (end 145.332 96.81) (width 0.3048) (layer F.Cu) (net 27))
 (segment (start 128.817 104.445) (end 128.822 104.44) (width 0.3048) (layer B.Cu) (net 9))
 (segment (start 128.822 104.44) (end 128.822 104.43) (width 0.3048) (layer B.Cu) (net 9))
 (segment (start 128.817 104.445) (end 128.817 106.985) (width 0.3048) (layer B.Cu) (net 9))
 (segment (start 128.817 101.905) (end 128.817 104.445) (width 0.3048) (layer B.Cu) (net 9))
 (segment (start 128.822 101.89) (end 128.822 104.43) (width 0.3048) (layer B.Cu) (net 9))
 (segment (start 133.902 89.19) (end 132.581 89.19) (width 0.3048) (layer B.Cu) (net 9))
 (segment (start 132.581 89.19) (end 130.854 90.917) (width 0.3048) (layer B.Cu) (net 9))
 (segment (start 130.854 90.917) (end 130.854 99.858) (width 0.3048) (layer B.Cu) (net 9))
 (segment (start 130.854 99.858) (end 128.822 101.89) (width 0.3048) (layer B.Cu) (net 9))
 (segment (start 128.817 106.985) (end 128.822 106.99) (width 0.3048) (layer B.Cu) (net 9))
 (segment (start 128.822 106.99) (end 128.822 112.05) (width 0.3048) (layer B.Cu) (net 9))
 (segment (start 128.817 106.985) (end 128.817 112.065) (width 0.3048) (layer B.Cu) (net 9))
 (segment (start 161.842 91.73) (end 168.192 91.73) (width 0.3048) (layer F.Cu) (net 30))
 (segment (start 133.902 84.11) (end 153.333 84.11) (width 0.3048) (layer B.Cu) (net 30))
 (segment (start 153.333 84.11) (end 154.654 85.4308) (width 0.3048) (layer B.Cu) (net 30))
 (segment (start 154.654 85.4308) (end 158.083 85.4308) (width 0.3048) (layer B.Cu) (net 30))
 (segment (start 158.083 85.4308) (end 161.842 89.19) (width 0.3048) (layer B.Cu) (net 30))
 (segment (start 161.842 89.19) (end 161.842 91.73) (width 0.3048) (layer B.Cu) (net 30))
 (via (at 161.842 91.73) (size 0.8128) (layers F.Cu B.Cu) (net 30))
 (segment (start 133.902 81.57) (end 134.054 81.57) (width 0.3048) (layer B.Cu) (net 31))
 (segment (start 133.902 81.57) (end 135.934 81.57) (width 0.3048) (layer F.Cu) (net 31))
 (segment (start 135.934 81.57) (end 137.585 83.221) (width 0.3048) (layer F.Cu) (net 31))
 (segment (start 137.585 83.221) (end 137.585 88.682) (width 0.3048) (layer F.Cu) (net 31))
 (segment (start 137.585 88.682) (end 141.903 93) (width 0.3048) (layer F.Cu) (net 31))
 (segment (start 141.903 93) (end 164.509 93) (width 0.3048) (layer F.Cu) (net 31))
 (segment (start 164.509 93) (end 165.779 94.27) (width 0.3048) (layer F.Cu) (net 31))
 (segment (start 165.779 94.27) (end 168.192 94.27) (width 0.3048) (layer F.Cu) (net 31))
 (segment (start 161.842 103.414) (end 161.837 103.419) (width 0.3048) (layer B.Cu) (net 8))
 (segment (start 161.837 103.419) (end 161.837 104.445) (width 0.3048) (layer B.Cu) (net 8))
 (segment (start 161.842 103.414) (end 161.842 102.398) (width 0.3048) (layer B.Cu) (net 8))
 (segment (start 161.842 102.398) (end 164.636 99.604) (width 0.3048) (layer B.Cu) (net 8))
 (segment (start 164.636 99.604) (end 164.636 92.492) (width 0.3048) (layer B.Cu) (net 8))
 (segment (start 164.636 92.492) (end 167.938 89.19) (width 0.3048) (layer B.Cu) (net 8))
 (segment (start 167.938 89.19) (end 168.192 89.19) (width 0.3048) (layer B.Cu) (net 8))
 (segment (start 161.842 104.43) (end 161.842 103.414) (width 0.3048) (layer B.Cu) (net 8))
 (segment (start 161.837 108.255) (end 161.842 108.26) (width 0.3048) (layer B.Cu) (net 8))
 (segment (start 161.842 108.26) (end 161.842 112.05) (width 0.3048) (layer B.Cu) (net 8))
 (segment (start 161.837 108.255) (end 161.837 112.065) (width 0.3048) (layer B.Cu) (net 8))
 (segment (start 161.837 104.445) (end 161.837 108.255) (width 0.3048) (layer B.Cu) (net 8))
 (segment (start 133.902 79.03) (end 136.188 79.03) (width 0.3048) (layer B.Cu) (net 8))
 (segment (start 136.188 79.03) (end 137.966 77.252) (width 0.3048) (layer B.Cu) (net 8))
 (segment (start 137.966 77.252) (end 158.032 77.252) (width 0.3048) (layer B.Cu) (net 8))
 (segment (start 158.032 77.252) (end 159.81 79.03) (width 0.3048) (layer B.Cu) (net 8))
 (segment (start 159.81 79.03) (end 159.81 81.824) (width 0.3048) (layer B.Cu) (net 8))
 (segment (start 159.81 81.824) (end 164.89 86.904) (width 0.3048) (layer B.Cu) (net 8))
 (segment (start 164.89 86.904) (end 164.89 88.428) (width 0.3048) (layer B.Cu) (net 8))
 (segment (start 164.89 88.428) (end 165.652 89.19) (width 0.3048) (layer B.Cu) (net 8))
 (segment (start 165.652 89.19) (end 168.192 89.19) (width 0.3048) (layer B.Cu) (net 8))
 (segment (start 146.602 117.13) (end 150.92 117.13) (width 0.8128) (layer F.Cu) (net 10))
 (segment (start 150.92 117.13) (end 153.46 114.59) (width 0.8128) (layer F.Cu) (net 10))
 (segment (start 153.46 114.59) (end 156.762 114.59) (width 0.8128) (layer F.Cu) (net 10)))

